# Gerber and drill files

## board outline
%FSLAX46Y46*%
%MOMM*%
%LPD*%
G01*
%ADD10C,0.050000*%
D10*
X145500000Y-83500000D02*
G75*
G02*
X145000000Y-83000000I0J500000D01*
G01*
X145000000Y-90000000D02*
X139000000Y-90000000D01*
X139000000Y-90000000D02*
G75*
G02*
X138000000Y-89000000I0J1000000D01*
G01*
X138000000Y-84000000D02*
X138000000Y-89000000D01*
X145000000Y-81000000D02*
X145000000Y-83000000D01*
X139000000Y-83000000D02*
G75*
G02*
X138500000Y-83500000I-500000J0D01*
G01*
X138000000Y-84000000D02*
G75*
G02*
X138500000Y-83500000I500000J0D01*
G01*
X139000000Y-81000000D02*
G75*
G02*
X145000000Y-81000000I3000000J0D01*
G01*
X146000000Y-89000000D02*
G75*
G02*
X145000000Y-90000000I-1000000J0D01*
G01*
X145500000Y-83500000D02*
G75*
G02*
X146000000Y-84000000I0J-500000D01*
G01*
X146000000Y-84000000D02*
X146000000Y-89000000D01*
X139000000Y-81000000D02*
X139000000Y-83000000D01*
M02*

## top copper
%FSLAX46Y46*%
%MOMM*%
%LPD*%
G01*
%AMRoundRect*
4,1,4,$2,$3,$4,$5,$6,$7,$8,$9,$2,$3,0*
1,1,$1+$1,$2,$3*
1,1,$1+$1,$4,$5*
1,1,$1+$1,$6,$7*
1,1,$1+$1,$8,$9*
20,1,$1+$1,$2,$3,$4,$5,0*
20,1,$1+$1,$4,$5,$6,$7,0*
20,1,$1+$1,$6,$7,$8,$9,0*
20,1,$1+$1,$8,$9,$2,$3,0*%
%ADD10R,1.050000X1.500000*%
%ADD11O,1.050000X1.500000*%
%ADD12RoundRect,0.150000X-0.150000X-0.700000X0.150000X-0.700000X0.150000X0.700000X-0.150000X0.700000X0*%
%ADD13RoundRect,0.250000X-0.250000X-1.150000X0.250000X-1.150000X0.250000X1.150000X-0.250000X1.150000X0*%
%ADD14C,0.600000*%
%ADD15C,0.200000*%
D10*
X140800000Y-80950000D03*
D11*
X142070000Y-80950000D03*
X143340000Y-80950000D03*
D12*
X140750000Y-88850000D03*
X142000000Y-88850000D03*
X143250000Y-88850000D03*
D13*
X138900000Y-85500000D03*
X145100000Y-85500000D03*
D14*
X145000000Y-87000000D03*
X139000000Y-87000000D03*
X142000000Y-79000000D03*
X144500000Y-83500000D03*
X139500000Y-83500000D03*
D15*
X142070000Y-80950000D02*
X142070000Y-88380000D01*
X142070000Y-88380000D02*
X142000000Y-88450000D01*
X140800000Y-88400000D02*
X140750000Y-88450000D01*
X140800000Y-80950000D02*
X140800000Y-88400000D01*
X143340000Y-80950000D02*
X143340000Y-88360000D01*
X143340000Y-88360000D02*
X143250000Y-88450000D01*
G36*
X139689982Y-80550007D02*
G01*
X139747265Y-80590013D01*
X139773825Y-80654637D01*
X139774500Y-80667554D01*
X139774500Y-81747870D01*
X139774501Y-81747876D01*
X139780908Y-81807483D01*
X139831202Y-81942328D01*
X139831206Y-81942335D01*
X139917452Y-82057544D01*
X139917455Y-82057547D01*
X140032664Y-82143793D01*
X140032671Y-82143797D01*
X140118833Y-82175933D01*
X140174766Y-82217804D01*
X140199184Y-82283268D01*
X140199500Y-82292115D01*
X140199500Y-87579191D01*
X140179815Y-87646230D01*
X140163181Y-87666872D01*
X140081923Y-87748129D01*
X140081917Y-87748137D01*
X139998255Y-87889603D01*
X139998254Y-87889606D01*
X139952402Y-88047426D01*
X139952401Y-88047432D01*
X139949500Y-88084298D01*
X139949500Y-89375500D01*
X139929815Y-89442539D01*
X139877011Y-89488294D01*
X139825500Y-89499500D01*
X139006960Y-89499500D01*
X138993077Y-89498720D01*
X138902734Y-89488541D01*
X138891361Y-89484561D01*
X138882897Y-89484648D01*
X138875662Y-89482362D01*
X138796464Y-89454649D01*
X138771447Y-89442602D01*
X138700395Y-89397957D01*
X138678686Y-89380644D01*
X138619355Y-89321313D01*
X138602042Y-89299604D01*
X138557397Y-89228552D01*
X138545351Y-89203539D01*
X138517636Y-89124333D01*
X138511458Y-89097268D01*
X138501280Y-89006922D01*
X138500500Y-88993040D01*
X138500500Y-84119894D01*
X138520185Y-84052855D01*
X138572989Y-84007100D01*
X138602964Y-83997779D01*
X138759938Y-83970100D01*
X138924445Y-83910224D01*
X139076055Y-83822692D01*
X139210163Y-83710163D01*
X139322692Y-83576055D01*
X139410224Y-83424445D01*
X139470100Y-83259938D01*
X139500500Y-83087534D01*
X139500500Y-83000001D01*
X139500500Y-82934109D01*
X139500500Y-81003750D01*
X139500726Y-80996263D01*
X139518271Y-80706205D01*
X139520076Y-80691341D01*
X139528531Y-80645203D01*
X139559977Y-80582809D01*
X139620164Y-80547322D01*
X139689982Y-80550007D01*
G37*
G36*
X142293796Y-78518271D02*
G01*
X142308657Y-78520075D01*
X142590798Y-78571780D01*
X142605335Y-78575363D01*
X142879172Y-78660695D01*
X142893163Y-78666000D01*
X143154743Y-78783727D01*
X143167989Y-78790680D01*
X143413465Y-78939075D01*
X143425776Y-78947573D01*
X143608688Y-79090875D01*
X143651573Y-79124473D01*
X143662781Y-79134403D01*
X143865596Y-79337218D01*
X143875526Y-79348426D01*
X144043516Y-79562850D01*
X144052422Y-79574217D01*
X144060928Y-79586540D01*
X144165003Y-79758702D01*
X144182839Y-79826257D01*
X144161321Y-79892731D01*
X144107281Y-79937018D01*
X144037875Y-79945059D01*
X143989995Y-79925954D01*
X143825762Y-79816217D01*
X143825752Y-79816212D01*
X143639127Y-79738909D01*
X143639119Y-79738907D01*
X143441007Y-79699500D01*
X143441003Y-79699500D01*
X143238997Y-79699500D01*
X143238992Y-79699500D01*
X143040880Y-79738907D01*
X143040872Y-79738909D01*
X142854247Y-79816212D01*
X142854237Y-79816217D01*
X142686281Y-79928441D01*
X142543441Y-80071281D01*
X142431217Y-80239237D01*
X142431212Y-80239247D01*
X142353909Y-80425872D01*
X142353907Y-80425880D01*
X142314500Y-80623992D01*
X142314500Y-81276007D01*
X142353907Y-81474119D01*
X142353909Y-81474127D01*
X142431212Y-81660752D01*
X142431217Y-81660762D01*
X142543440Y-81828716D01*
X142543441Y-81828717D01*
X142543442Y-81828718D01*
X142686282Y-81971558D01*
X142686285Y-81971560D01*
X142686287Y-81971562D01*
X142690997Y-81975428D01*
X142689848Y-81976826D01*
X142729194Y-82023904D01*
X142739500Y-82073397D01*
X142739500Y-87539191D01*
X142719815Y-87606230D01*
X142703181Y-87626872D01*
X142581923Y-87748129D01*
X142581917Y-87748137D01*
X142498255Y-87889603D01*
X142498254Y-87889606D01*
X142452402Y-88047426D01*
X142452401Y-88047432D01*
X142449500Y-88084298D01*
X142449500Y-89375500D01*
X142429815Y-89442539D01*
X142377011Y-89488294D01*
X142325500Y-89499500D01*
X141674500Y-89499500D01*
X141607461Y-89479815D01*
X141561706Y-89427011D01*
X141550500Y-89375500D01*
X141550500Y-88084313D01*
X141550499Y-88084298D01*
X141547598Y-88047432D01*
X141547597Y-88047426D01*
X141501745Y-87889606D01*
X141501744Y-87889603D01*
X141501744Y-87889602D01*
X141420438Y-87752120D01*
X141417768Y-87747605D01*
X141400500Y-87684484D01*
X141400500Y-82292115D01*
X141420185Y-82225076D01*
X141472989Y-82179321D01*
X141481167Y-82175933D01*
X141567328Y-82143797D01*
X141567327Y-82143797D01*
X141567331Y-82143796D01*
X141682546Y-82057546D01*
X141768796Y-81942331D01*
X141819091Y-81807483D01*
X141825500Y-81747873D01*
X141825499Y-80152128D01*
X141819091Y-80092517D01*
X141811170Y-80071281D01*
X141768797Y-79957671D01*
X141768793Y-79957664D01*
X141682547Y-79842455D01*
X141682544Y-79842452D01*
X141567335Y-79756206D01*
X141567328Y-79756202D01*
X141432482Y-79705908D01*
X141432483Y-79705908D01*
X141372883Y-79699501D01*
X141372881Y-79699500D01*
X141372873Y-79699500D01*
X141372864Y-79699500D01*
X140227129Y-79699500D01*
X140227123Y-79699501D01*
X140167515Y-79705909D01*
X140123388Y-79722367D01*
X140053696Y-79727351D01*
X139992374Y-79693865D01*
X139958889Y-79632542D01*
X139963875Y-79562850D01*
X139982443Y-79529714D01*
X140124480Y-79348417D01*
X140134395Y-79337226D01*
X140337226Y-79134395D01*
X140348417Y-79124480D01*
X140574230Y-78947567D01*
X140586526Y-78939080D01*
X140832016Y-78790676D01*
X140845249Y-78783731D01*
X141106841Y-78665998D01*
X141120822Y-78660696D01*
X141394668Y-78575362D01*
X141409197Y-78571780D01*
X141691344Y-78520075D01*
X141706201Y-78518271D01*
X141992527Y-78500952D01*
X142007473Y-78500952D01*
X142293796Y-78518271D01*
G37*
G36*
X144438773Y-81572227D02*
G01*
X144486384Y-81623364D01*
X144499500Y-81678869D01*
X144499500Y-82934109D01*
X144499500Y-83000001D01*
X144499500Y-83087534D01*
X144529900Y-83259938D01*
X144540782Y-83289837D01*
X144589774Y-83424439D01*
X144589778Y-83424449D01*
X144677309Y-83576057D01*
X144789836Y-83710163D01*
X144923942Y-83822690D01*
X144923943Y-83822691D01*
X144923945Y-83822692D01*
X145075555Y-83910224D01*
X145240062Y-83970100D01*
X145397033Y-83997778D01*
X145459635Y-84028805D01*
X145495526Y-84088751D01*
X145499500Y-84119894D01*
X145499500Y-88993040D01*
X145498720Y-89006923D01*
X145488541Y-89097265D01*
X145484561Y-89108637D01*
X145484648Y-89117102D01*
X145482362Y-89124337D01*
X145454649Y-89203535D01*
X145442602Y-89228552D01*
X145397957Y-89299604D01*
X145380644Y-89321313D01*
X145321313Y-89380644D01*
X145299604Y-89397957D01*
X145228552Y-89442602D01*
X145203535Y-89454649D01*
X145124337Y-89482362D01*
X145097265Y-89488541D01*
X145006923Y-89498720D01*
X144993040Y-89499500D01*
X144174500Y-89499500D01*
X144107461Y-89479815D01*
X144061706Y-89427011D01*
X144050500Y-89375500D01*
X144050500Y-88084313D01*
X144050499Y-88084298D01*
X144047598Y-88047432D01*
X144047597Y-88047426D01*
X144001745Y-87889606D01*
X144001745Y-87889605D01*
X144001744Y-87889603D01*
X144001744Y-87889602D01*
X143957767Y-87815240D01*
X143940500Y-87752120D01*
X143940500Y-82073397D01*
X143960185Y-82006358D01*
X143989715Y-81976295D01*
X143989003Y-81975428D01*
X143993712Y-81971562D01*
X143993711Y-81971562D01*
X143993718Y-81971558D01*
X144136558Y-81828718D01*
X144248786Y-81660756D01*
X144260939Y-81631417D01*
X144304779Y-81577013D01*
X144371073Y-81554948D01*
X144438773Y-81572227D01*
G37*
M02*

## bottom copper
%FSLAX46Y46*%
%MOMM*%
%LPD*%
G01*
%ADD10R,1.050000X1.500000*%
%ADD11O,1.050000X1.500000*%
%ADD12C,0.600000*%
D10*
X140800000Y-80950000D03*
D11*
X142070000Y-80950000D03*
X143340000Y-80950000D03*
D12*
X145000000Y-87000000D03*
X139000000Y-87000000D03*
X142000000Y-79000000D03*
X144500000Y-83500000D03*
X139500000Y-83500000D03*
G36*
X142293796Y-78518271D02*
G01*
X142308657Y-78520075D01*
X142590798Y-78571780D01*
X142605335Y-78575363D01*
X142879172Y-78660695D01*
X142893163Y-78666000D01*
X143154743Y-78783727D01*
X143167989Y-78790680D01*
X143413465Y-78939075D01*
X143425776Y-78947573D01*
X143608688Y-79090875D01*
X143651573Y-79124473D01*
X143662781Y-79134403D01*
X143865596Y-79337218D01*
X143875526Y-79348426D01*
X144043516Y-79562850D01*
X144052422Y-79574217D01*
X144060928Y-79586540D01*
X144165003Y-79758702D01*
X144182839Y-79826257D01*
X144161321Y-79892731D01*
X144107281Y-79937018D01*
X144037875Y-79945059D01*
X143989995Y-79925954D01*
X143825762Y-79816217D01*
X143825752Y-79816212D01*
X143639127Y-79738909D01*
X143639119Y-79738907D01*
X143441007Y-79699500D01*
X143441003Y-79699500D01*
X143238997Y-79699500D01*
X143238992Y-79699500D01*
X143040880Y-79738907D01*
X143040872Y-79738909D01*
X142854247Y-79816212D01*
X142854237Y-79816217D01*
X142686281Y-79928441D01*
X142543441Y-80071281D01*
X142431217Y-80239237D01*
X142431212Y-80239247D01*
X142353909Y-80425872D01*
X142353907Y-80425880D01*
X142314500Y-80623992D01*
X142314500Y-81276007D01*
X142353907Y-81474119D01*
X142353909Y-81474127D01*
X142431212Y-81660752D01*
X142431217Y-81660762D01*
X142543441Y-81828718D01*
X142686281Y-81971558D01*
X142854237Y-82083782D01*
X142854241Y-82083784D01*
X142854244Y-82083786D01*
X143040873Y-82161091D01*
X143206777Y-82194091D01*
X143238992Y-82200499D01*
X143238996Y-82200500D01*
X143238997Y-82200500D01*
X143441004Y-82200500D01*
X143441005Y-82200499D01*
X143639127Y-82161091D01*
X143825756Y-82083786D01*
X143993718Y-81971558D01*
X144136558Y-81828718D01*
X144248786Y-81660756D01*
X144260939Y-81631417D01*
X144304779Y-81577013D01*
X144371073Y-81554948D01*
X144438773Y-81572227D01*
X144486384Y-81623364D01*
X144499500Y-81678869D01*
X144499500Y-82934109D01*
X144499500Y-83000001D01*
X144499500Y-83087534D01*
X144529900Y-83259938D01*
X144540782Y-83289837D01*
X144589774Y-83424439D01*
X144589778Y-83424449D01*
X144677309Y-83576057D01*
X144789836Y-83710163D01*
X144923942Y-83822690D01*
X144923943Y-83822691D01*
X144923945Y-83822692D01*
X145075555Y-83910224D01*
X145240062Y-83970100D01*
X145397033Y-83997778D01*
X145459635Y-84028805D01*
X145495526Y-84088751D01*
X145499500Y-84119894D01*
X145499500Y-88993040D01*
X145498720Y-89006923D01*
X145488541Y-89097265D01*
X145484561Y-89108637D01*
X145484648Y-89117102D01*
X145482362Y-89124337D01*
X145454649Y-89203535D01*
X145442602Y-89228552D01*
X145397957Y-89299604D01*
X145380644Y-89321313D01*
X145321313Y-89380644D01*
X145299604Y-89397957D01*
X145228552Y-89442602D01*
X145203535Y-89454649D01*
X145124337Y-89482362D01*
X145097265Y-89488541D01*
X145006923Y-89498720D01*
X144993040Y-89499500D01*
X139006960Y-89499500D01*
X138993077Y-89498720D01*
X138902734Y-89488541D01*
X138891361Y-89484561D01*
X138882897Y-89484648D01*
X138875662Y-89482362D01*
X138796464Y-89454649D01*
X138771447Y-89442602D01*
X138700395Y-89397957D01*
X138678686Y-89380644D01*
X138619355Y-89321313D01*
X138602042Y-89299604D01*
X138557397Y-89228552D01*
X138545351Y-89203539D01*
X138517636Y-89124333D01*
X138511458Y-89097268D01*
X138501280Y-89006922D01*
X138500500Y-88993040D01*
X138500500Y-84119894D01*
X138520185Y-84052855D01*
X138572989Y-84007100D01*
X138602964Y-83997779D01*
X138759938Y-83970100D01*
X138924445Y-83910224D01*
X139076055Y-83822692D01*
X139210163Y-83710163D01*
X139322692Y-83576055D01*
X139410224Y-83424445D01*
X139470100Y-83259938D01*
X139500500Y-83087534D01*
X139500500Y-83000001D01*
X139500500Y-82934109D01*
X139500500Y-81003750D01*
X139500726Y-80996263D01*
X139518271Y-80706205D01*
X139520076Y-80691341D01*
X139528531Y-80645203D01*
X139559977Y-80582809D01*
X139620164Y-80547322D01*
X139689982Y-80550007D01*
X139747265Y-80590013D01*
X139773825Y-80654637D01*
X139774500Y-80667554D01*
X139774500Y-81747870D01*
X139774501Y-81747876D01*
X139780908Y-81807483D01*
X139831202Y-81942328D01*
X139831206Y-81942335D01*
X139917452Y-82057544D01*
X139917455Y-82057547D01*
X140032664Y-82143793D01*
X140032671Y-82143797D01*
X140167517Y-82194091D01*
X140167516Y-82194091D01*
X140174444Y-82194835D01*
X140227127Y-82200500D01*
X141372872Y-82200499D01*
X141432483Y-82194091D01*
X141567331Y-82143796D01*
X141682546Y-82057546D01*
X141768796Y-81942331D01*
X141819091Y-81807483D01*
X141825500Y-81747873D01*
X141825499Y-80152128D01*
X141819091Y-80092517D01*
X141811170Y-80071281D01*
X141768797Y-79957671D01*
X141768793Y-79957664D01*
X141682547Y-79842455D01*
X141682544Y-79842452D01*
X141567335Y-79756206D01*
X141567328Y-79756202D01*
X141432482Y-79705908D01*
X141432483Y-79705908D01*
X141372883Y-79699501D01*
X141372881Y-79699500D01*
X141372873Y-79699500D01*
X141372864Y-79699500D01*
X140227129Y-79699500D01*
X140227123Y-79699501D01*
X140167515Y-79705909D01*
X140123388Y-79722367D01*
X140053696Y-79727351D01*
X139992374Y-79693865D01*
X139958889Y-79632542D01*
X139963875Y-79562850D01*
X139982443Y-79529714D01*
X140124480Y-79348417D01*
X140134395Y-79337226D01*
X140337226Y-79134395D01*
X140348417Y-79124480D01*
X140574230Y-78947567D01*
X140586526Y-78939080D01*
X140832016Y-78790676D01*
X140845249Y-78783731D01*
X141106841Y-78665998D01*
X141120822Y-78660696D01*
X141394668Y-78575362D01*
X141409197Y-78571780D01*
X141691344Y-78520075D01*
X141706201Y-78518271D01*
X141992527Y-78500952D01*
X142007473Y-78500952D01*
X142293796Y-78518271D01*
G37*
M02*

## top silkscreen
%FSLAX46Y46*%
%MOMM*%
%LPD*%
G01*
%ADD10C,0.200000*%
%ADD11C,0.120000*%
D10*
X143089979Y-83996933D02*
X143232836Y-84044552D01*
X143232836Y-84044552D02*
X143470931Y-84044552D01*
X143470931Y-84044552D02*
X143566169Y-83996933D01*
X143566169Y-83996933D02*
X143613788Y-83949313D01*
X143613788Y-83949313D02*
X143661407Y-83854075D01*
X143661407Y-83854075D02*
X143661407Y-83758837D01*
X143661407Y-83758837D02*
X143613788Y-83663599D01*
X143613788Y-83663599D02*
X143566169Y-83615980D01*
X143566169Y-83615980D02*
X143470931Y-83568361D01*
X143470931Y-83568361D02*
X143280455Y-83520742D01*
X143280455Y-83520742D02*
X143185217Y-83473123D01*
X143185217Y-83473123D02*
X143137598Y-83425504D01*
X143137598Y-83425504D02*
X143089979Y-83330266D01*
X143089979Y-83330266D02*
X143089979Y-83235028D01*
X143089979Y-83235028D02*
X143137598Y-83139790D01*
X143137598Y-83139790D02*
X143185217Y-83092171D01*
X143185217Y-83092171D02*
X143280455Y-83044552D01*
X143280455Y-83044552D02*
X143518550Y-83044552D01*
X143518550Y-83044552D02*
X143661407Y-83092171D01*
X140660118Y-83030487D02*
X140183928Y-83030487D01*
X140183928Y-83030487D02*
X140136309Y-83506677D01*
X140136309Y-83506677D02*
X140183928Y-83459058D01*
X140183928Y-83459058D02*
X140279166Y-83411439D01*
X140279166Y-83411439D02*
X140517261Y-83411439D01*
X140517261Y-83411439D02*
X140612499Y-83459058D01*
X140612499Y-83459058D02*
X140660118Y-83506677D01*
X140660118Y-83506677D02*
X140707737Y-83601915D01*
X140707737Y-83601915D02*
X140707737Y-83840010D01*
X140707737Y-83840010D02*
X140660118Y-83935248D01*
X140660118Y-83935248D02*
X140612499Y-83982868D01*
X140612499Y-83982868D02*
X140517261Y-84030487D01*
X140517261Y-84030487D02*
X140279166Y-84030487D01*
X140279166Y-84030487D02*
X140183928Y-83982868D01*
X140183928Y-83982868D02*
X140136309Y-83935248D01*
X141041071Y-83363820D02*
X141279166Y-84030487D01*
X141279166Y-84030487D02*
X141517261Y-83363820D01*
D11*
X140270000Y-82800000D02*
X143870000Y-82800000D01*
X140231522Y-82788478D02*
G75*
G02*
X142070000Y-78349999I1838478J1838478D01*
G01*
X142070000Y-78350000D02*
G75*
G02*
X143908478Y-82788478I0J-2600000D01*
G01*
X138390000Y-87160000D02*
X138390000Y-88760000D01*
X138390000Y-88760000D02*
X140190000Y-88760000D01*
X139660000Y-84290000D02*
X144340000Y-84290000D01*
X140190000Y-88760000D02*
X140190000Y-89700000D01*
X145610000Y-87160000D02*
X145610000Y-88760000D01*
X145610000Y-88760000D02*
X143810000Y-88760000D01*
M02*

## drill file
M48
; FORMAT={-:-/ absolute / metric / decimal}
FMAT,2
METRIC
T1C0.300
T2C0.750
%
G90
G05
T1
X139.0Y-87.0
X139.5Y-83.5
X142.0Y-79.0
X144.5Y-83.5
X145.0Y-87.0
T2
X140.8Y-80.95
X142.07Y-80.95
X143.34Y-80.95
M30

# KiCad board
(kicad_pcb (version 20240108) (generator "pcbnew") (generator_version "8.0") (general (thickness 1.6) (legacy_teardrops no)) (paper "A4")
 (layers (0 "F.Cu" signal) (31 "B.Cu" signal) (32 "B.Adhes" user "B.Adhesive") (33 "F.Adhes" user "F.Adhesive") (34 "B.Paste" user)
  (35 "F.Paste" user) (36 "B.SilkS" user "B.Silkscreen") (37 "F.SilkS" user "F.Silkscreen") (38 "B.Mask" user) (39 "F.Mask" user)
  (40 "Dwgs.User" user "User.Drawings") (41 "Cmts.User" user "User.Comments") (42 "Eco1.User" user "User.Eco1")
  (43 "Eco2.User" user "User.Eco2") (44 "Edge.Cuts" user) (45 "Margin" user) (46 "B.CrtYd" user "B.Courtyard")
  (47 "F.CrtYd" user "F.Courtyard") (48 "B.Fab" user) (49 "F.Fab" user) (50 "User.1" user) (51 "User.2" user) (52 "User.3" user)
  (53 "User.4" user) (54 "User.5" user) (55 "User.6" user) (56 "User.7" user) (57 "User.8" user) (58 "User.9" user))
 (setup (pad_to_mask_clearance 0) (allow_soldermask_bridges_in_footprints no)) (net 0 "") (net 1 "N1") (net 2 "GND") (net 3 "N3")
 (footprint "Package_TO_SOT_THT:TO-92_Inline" (layer "F.Cu") (at 140.8 80.95)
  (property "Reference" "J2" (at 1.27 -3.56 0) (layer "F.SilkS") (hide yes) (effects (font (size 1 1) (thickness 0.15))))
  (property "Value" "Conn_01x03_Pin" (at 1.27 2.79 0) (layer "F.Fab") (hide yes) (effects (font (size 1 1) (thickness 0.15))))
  (fp_line (start -0.53 1.85) (end 3.07 1.85) (stroke (width 0.12) (type solid)) (layer "F.SilkS"))
  (fp_arc (start -0.568478 1.838478) (mid -1.132087 -0.994977) (end 1.27 -2.6) (stroke (width 0.12) (type solid)) (layer "F.SilkS"))
  (fp_arc (start 1.27 -2.6) (mid 3.672087 -0.994977) (end 3.108478 1.838478) (stroke (width 0.12) (type solid)) (layer "F.SilkS"))
  (pad "1" thru_hole rect (at 0 0) (size 1.05 1.5) (drill 0.75) (layers "*.Cu" "*.Mask") (remove_unused_layers no) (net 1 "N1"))
  (pad "2" thru_hole oval (at 1.27 0) (size 1.05 1.5) (drill 0.75) (layers "*.Cu" "*.Mask") (remove_unused_layers no) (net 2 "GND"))
  (pad "3" thru_hole oval (at 2.54 0) (size 1.05 1.5) (drill 0.75) (layers "*.Cu" "*.Mask") (remove_unused_layers no) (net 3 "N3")))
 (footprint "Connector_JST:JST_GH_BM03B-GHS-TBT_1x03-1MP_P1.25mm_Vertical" (layer "F.Cu") (at 142 86.9)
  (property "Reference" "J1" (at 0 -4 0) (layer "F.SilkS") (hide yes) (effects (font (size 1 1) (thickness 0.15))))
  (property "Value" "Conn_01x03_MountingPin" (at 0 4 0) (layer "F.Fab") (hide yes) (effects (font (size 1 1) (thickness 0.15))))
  (fp_line (start -3.61 0.26) (end -3.61 1.86) (stroke (width 0.12) (type solid)) (layer "F.SilkS"))
  (fp_line (start -3.61 1.86) (end -1.81 1.86) (stroke (width 0.12) (type solid)) (layer "F.SilkS"))
  (fp_line (start -2.34 -2.61) (end 2.34 -2.61) (stroke (width 0.12) (type solid)) (layer "F.SilkS"))
  (fp_line (start -1.81 1.86) (end -1.81 2.8) (stroke (width 0.12) (type solid)) (layer "F.SilkS"))
  (fp_line (start 3.61 0.26) (end 3.61 1.86) (stroke (width 0.12) (type solid)) (layer "F.SilkS"))
  (fp_line (start 3.61 1.86) (end 1.81 1.86) (stroke (width 0.12) (type solid)) (layer "F.SilkS"))
  (pad "1" smd roundrect (at -1.25 1.95) (size 0.6 1.7) (layers "F.Cu" "F.Paste" "F.Mask") (roundrect_rratio 0.25) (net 1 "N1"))
  (pad "2" smd roundrect (at 0 1.95) (size 0.6 1.7) (layers "F.Cu" "F.Paste" "F.Mask") (roundrect_rratio 0.25) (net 2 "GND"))
  (pad "3" smd roundrect (at 1.25 1.95) (size 0.6 1.7) (layers "F.Cu" "F.Paste" "F.Mask") (roundrect_rratio 0.25) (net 3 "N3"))
  (pad "MP" smd roundrect (at -3.1 -1.4) (size 1 2.8) (layers "F.Cu" "F.Paste" "F.Mask") (roundrect_rratio 0.25) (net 2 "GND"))
  (pad "MP" smd roundrect (at 3.1 -1.4) (size 1 2.8) (layers "F.Cu" "F.Paste" "F.Mask") (roundrect_rratio 0.25) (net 2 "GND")))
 (gr_arc (start 145.5 83.5) (mid 145.146447 83.353553) (end 145 83) (stroke (width 0.05) (type default)) (layer "Edge.Cuts"))
 (gr_line (start 145 90) (end 139 90) (stroke (width 0.05) (type default)) (layer "Edge.Cuts"))
 (gr_arc (start 139 90) (mid 138.292893 89.707107) (end 138 89) (stroke (width 0.05) (type default)) (layer "Edge.Cuts"))
 (gr_line (start 138 84) (end 138 89) (stroke (width 0.05) (type default)) (layer "Edge.Cuts"))
 (gr_line (start 145 81) (end 145 83) (stroke (width 0.05) (type default)) (layer "Edge.Cuts"))
 (gr_arc (start 139 83) (mid 138.853553 83.353553) (end 138.5 83.5) (stroke (width 0.05) (type default)) (layer "Edge.Cuts"))
 (gr_arc (start 138 84) (mid 138.146447 83.646447) (end 138.5 83.5) (stroke (width 0.05) (type default)) (layer "Edge.Cuts"))
 (gr_arc (start 139 81) (mid 142 78) (end 145 81) (stroke (width 0.05) (type default)) (layer "Edge.Cuts"))
 (gr_arc (start 146 89) (mid 145.707107 89.707107) (end 145 90) (stroke (width 0.05) (type default)) (layer "Edge.Cuts"))
 (gr_arc (start 145.5 83.5) (mid 145.853553 83.646447) (end 146 84) (stroke (width 0.05) (type default)) (layer "Edge.Cuts"))
 (gr_line (start 146 84) (end 146 89) (stroke (width 0.05) (type default)) (layer "Edge.Cuts"))
 (gr_line (start 139 81) (end 139 83) (stroke (width 0.05) (type default)) (layer "Edge.Cuts"))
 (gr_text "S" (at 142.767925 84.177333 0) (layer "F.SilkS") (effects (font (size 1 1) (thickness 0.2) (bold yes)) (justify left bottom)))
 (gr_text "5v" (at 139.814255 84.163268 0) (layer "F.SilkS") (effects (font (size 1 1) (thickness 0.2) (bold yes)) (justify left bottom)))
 (segment (start 142.07 80.95) (end 142.07 88.38) (width 0.2) (layer "F.Cu") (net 2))
 (segment (start 142.07 88.38) (end 142 88.45) (width 0.2) (layer "F.Cu") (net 2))
 (via (at 145 87) (size 0.6) (drill 0.3) (layers "F.Cu" "B.Cu") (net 2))
 (via (at 139 87) (size 0.6) (drill 0.3) (layers "F.Cu" "B.Cu") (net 2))
 (via (at 142 79) (size 0.6) (drill 0.3) (layers "F.Cu" "B.Cu") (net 2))
 (via (at 144.5 83.5) (size 0.6) (drill 0.3) (layers "F.Cu" "B.Cu") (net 2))
 (via (at 139.5 83.5) (size 0.6) (drill 0.3) (layers "F.Cu" "B.Cu") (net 2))
 (segment (start 140.8 88.4) (end 140.75 88.45) (width 0.2) (layer "F.Cu") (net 1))
 (segment (start 140.8 80.95) (end 140.8 88.4) (width 0.2) (layer "F.Cu") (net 1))
 (segment (start 143.34 80.95) (end 143.34 88.36) (width 0.2) (layer "F.Cu") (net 3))
 (segment (start 143.34 88.36) (end 143.25 88.45) (width 0.2) (layer "F.Cu") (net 3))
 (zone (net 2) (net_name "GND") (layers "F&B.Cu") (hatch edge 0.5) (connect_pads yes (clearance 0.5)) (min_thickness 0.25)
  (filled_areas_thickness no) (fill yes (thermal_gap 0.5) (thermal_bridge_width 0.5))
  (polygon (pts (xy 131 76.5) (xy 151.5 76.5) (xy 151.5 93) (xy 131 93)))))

